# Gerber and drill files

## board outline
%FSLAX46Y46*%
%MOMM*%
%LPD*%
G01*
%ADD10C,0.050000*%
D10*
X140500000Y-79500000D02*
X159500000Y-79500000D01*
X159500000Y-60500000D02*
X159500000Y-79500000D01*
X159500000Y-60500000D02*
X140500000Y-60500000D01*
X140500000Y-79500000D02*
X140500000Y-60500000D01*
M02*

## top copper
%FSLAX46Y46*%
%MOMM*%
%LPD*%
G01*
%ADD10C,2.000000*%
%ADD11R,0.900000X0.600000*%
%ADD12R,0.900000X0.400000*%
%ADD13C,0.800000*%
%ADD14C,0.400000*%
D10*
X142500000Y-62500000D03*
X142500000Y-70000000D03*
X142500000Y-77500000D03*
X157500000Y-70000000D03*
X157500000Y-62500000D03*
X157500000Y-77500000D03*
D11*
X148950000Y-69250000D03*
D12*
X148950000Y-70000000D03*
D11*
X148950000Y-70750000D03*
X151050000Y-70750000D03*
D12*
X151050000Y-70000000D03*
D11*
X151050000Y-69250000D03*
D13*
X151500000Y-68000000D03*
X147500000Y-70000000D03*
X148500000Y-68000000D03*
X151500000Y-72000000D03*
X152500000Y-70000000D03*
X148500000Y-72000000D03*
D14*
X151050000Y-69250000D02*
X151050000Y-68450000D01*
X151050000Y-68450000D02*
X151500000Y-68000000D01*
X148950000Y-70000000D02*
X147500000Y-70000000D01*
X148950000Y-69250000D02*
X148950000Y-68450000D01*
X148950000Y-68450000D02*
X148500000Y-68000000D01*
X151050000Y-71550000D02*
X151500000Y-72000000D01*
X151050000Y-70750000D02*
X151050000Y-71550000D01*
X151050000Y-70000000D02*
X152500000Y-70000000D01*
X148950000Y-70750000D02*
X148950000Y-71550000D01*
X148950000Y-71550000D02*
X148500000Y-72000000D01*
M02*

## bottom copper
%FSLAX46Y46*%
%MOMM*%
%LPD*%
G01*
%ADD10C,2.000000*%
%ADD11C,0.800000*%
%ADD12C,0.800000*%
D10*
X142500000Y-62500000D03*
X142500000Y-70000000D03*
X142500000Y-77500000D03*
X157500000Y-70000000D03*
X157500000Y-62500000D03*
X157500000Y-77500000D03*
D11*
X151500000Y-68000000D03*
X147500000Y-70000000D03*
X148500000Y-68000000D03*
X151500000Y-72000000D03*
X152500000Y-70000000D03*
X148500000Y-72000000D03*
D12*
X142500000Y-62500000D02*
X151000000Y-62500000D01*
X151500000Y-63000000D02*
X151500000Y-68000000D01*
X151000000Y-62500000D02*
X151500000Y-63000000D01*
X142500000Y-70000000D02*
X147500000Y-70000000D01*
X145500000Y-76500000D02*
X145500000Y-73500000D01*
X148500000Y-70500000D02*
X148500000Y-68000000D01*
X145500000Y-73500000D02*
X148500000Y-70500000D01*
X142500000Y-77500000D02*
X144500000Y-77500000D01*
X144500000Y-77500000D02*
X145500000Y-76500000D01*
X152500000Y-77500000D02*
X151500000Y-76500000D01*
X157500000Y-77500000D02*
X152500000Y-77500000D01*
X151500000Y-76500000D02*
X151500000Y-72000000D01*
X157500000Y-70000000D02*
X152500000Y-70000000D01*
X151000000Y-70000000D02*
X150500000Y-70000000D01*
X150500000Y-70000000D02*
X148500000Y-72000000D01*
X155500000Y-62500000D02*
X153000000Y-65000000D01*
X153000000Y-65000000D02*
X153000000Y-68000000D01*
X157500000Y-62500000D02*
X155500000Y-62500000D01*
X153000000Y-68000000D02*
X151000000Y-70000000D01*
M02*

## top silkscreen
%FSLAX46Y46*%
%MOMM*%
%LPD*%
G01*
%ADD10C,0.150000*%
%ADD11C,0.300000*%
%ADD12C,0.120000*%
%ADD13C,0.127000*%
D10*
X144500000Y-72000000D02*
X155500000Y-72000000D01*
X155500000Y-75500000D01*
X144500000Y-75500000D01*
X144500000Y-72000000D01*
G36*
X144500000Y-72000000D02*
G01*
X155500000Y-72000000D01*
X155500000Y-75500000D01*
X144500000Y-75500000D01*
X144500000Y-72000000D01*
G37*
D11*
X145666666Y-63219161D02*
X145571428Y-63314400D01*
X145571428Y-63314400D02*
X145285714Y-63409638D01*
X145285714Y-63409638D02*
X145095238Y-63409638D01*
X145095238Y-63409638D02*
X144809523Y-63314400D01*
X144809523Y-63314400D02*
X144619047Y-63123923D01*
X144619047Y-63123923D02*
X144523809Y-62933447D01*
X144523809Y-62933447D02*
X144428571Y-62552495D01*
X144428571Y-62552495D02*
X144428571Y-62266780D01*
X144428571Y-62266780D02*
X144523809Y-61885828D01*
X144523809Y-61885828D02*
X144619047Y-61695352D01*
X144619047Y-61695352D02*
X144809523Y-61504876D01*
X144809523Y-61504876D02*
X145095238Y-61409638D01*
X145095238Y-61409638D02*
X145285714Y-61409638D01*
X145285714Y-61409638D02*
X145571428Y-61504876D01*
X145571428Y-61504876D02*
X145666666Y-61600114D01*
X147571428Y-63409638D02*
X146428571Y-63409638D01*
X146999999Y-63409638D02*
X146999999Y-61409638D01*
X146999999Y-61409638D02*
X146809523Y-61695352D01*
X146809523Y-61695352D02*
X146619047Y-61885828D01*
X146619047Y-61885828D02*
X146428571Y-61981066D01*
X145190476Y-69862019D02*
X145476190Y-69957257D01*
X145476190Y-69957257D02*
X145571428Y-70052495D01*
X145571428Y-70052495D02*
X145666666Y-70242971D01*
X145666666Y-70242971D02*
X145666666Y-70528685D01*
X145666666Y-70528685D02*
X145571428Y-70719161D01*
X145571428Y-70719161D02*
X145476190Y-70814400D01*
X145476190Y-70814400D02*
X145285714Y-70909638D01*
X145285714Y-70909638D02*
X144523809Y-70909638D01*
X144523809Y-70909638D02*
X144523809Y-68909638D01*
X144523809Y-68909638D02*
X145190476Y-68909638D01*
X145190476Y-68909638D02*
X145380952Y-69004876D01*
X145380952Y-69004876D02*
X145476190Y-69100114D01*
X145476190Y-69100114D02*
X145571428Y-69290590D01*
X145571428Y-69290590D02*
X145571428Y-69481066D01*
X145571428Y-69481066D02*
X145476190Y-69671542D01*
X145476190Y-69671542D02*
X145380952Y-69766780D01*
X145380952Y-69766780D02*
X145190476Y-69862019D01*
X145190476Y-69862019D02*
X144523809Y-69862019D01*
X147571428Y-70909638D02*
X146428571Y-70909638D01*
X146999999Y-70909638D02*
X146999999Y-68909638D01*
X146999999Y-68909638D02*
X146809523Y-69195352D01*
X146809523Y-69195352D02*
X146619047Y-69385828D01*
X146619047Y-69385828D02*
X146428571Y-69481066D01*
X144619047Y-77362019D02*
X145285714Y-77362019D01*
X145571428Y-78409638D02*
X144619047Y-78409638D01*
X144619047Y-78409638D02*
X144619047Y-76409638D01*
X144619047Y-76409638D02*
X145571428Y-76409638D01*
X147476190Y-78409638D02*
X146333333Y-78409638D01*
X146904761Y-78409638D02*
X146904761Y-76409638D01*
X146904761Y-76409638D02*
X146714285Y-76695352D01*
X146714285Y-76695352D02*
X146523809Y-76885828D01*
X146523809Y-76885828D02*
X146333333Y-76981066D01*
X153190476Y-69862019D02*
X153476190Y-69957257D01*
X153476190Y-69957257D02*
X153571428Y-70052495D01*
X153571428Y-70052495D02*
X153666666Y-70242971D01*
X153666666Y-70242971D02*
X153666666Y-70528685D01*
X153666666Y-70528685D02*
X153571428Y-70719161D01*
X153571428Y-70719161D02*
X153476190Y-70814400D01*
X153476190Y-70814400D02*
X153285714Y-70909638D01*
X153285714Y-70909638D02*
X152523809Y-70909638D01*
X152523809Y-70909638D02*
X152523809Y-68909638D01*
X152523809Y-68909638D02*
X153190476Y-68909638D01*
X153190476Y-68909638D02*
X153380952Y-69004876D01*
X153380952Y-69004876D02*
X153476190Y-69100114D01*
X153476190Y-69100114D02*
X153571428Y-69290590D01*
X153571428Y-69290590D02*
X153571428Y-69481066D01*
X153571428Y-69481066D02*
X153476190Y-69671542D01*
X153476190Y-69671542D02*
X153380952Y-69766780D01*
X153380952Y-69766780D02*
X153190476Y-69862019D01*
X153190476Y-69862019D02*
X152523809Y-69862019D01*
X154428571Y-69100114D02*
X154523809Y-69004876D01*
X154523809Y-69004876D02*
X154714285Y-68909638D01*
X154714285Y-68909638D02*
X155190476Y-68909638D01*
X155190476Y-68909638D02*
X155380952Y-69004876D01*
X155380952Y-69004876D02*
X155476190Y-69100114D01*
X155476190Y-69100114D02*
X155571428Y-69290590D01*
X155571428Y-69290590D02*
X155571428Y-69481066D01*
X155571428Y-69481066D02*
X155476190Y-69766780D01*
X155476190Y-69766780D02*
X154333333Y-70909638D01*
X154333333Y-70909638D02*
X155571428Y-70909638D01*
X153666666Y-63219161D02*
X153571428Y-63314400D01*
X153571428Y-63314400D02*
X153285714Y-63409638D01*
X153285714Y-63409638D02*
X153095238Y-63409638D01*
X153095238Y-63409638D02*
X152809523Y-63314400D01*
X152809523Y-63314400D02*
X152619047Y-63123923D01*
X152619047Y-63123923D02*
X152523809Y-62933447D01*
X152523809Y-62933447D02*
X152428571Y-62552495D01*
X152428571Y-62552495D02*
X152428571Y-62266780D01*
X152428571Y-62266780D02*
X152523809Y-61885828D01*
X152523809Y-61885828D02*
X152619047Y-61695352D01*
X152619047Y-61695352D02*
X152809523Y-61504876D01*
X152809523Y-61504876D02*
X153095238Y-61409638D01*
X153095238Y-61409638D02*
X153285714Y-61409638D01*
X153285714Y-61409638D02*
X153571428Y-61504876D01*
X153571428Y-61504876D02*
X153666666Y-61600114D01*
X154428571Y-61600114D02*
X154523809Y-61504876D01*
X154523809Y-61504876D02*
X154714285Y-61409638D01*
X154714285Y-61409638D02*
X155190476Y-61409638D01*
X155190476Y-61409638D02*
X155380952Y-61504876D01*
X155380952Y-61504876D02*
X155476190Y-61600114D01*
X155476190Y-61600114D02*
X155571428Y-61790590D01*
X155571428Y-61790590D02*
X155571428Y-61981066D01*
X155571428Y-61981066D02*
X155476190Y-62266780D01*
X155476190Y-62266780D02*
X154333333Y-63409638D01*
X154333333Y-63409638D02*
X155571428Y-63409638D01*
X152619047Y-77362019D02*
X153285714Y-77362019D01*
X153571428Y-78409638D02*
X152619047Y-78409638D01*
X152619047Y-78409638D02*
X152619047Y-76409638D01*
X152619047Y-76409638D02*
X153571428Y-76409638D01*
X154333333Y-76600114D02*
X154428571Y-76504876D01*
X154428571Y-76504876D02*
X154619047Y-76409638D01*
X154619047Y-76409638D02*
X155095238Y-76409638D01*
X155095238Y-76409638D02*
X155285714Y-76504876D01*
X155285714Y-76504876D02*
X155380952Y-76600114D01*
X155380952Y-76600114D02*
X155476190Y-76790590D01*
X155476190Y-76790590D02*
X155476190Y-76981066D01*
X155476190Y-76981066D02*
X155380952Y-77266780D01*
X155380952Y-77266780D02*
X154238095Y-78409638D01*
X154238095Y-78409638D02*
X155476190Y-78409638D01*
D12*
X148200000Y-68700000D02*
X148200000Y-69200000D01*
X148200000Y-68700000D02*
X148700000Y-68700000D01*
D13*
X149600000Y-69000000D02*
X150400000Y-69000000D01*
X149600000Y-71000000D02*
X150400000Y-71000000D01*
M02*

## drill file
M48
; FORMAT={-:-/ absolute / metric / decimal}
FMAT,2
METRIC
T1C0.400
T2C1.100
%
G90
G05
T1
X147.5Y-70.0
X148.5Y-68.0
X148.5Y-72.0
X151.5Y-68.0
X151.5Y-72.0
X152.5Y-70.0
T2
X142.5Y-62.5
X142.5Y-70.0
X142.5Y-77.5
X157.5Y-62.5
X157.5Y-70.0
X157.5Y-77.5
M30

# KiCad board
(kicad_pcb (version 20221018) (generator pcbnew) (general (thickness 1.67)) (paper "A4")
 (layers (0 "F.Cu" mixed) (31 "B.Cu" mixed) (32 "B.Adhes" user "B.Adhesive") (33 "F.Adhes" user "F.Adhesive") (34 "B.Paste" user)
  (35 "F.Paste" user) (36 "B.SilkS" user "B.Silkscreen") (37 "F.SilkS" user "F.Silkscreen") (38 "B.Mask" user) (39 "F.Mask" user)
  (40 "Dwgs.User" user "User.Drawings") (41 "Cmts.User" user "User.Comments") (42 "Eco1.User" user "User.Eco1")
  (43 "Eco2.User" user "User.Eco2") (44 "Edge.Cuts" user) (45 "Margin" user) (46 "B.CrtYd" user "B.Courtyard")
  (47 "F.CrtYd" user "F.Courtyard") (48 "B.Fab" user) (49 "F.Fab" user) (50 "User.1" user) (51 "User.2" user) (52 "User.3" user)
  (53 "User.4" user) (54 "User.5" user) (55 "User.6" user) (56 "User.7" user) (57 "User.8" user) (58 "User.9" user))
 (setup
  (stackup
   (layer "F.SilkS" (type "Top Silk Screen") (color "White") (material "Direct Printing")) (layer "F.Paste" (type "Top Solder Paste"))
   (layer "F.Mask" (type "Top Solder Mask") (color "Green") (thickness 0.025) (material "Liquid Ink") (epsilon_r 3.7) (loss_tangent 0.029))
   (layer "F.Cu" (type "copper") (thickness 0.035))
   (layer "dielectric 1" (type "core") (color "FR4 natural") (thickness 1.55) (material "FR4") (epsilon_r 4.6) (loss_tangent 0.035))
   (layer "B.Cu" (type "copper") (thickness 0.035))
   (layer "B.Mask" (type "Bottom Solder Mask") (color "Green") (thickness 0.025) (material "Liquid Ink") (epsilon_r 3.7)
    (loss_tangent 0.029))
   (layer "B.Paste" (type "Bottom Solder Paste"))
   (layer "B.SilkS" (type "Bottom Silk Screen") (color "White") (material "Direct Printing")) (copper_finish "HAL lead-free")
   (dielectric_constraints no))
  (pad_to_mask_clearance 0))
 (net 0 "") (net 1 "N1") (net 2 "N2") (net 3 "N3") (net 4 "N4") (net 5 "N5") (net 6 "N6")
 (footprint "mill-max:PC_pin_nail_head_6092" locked (layer "F.Cu") (at 142.5 62.5)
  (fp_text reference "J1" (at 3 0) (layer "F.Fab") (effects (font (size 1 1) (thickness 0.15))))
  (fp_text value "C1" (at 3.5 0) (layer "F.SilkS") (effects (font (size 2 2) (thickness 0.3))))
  (pad "1" thru_hole circle locked (at 0 0) (size 2 2) (drill 1.1) (layers "*.Cu" "*.Mask") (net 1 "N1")))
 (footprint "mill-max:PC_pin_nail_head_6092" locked (layer "F.Cu") (at 142.5 70)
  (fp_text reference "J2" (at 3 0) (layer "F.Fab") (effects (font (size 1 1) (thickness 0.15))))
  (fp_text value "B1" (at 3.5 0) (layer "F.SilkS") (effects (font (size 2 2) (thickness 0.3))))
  (pad "1" thru_hole circle locked (at 0 0) (size 2 2) (drill 1.1) (layers "*.Cu" "*.Mask") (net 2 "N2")))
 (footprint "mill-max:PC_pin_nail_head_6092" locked (layer "F.Cu") (at 142.5 77.5)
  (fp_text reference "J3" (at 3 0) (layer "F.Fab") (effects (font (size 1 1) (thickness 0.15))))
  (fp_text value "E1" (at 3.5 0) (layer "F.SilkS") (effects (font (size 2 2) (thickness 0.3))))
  (pad "1" thru_hole circle locked (at 0 0) (size 2 2) (drill 1.1) (layers "*.Cu" "*.Mask") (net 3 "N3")))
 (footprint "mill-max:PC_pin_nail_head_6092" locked (layer "F.Cu") (at 157.5 70)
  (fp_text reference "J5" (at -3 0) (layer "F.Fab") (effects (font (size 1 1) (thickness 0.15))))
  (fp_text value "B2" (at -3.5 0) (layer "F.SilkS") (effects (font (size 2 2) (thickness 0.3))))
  (pad "1" thru_hole circle locked (at 0 0) (size 2 2) (drill 1.1) (layers "*.Cu" "*.Mask") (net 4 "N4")))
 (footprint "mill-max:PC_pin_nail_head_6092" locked (layer "F.Cu") (at 157.5 62.5)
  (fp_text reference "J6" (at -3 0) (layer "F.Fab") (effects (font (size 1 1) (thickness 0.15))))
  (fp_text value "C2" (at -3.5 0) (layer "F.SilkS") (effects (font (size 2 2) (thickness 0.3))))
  (pad "1" thru_hole circle locked (at 0 0) (size 2 2) (drill 1.1) (layers "*.Cu" "*.Mask") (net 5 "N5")))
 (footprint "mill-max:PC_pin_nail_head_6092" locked (layer "F.Cu") (at 157.5 77.5)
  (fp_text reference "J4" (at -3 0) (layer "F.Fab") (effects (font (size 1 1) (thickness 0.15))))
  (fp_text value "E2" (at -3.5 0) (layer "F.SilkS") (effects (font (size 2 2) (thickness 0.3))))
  (pad "1" thru_hole circle locked (at 0 0) (size 2 2) (drill 1.1) (layers "*.Cu" "*.Mask") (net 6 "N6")))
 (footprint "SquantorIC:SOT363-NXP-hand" (layer "F.Cu") (at 150 70)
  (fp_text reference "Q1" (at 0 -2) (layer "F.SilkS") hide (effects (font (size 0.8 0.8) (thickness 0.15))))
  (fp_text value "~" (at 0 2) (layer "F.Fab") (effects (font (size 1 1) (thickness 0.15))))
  (fp_line (start -1.8 -1.3) (end -1.8 -0.8) (stroke (width 0.12) (type solid)) (layer "F.SilkS"))
  (fp_line (start -1.8 -1.3) (end -1.3 -1.3) (stroke (width 0.12) (type solid)) (layer "F.SilkS"))
  (fp_line (start -0.4 -1) (end 0.4 -1) (stroke (width 0.127) (type solid)) (layer "F.SilkS"))
  (fp_line (start -0.4 1) (end 0.4 1) (stroke (width 0.127) (type solid)) (layer "F.SilkS"))
  (pad "1" smd rect (at -1.05 -0.75 270) (size 0.6 0.9) (layers "F.Cu" "F.Paste" "F.Mask") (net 3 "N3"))
  (pad "2" smd rect (at -1.05 0 270) (size 0.4 0.9) (layers "F.Cu" "F.Paste" "F.Mask") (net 2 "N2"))
  (pad "3" smd rect (at -1.05 0.75 270) (size 0.6 0.9) (layers "F.Cu" "F.Paste" "F.Mask") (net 5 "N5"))
  (pad "4" smd rect (at 1.05 0.75 270) (size 0.6 0.9) (layers "F.Cu" "F.Paste" "F.Mask") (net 6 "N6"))
  (pad "5" smd rect (at 1.05 0 270) (size 0.4 0.9) (layers "F.Cu" "F.Paste" "F.Mask") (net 4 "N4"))
  (pad "6" smd rect (at 1.05 -0.75 270) (size 0.6 0.9) (layers "F.Cu" "F.Paste" "F.Mask") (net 1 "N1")))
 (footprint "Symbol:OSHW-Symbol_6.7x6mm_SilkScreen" (layer "B.Cu") (at 150 74.8 180)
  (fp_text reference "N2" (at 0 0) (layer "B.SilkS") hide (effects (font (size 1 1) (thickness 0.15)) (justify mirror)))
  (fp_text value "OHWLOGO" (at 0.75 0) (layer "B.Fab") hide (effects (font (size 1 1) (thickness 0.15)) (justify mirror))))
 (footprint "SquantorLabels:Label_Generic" (layer "B.Cu") (at 150.9 78.5 180)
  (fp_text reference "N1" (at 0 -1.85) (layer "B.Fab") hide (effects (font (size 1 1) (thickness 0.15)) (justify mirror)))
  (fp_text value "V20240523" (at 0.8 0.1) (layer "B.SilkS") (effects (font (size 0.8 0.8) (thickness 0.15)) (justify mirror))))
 (gr_rect (start 144.5 72) (end 155.5 75.5) (stroke (width 0.15) (type solid)) (fill solid) (layer "F.SilkS"))
 (gr_line (start 140.5 79.5) (end 159.5 79.5) (stroke (width 0.05) (type solid)) (layer "Edge.Cuts"))
 (gr_line (start 159.5 60.5) (end 159.5 79.5) (stroke (width 0.05) (type solid)) (layer "Edge.Cuts"))
 (gr_line (start 159.5 60.5) (end 140.5 60.5) (stroke (width 0.05) (type solid)) (layer "Edge.Cuts"))
 (gr_line (start 140.5 79.5) (end 140.5 60.5) (stroke (width 0.05) (type solid)) (layer "Edge.Cuts"))
 (segment (start 151.05 69.25) (end 151.05 68.45) (width 0.4) (layer "F.Cu") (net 1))
 (segment (start 151.05 68.45) (end 151.5 68) (width 0.4) (layer "F.Cu") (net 1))
 (via (at 151.5 68) (size 0.8) (drill 0.4) (layers "F.Cu" "B.Cu") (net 1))
 (segment (start 142.5 62.5) (end 151 62.5) (width 0.8) (layer "B.Cu") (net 1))
 (segment (start 151.5 63) (end 151.5 68) (width 0.8) (layer "B.Cu") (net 1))
 (segment (start 151 62.5) (end 151.5 63) (width 0.8) (layer "B.Cu") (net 1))
 (segment (start 148.95 70) (end 147.5 70) (width 0.4) (layer "F.Cu") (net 2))
 (via (at 147.5 70) (size 0.8) (drill 0.4) (layers "F.Cu" "B.Cu") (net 2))
 (segment (start 142.5 70) (end 147.5 70) (width 0.8) (layer "B.Cu") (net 2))
 (segment (start 148.95 69.25) (end 148.95 68.45) (width 0.4) (layer "F.Cu") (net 3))
 (segment (start 148.95 68.45) (end 148.5 68) (width 0.4) (layer "F.Cu") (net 3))
 (via (at 148.5 68) (size 0.8) (drill 0.4) (layers "F.Cu" "B.Cu") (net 3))
 (segment (start 145.5 76.5) (end 145.5 73.5) (width 0.8) (layer "B.Cu") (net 3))
 (segment (start 148.5 70.5) (end 148.5 68) (width 0.8) (layer "B.Cu") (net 3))
 (segment (start 145.5 73.5) (end 148.5 70.5) (width 0.8) (layer "B.Cu") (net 3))
 (segment (start 142.5 77.5) (end 144.5 77.5) (width 0.8) (layer "B.Cu") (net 3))
 (segment (start 144.5 77.5) (end 145.5 76.5) (width 0.8) (layer "B.Cu") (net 3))
 (segment (start 151.05 71.55) (end 151.5 72) (width 0.4) (layer "F.Cu") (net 6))
 (segment (start 151.05 70.75) (end 151.05 71.55) (width 0.4) (layer "F.Cu") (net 6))
 (via (at 151.5 72) (size 0.8) (drill 0.4) (layers "F.Cu" "B.Cu") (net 6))
 (segment (start 152.5 77.5) (end 151.5 76.5) (width 0.8) (layer "B.Cu") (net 6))
 (segment (start 157.5 77.5) (end 152.5 77.5) (width 0.8) (layer "B.Cu") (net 6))
 (segment (start 151.5 76.5) (end 151.5 72) (width 0.8) (layer "B.Cu") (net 6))
 (segment (start 151.05 70) (end 152.5 70) (width 0.4) (layer "F.Cu") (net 4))
 (via (at 152.5 70) (size 0.8) (drill 0.4) (layers "F.Cu" "B.Cu") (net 4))
 (segment (start 157.5 70) (end 152.5 70) (width 0.8) (layer "B.Cu") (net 4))
 (segment (start 148.95 70.75) (end 148.95 71.55) (width 0.4) (layer "F.Cu") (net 5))
 (segment (start 148.95 71.55) (end 148.5 72) (width 0.4) (layer "F.Cu") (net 5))
 (via (at 148.5 72) (size 0.8) (drill 0.4) (layers "F.Cu" "B.Cu") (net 5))
 (segment (start 151 70) (end 150.5 70) (width 0.8) (layer "B.Cu") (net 5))
 (segment (start 150.5 70) (end 148.5 72) (width 0.8) (layer "B.Cu") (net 5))
 (segment (start 155.5 62.5) (end 153 65) (width 0.8) (layer "B.Cu") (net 5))
 (segment (start 153 65) (end 153 68) (width 0.8) (layer "B.Cu") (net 5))
 (segment (start 157.5 62.5) (end 155.5 62.5) (width 0.8) (layer "B.Cu") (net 5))
 (segment (start 153 68) (end 151 70) (width 0.8) (layer "B.Cu") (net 5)))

